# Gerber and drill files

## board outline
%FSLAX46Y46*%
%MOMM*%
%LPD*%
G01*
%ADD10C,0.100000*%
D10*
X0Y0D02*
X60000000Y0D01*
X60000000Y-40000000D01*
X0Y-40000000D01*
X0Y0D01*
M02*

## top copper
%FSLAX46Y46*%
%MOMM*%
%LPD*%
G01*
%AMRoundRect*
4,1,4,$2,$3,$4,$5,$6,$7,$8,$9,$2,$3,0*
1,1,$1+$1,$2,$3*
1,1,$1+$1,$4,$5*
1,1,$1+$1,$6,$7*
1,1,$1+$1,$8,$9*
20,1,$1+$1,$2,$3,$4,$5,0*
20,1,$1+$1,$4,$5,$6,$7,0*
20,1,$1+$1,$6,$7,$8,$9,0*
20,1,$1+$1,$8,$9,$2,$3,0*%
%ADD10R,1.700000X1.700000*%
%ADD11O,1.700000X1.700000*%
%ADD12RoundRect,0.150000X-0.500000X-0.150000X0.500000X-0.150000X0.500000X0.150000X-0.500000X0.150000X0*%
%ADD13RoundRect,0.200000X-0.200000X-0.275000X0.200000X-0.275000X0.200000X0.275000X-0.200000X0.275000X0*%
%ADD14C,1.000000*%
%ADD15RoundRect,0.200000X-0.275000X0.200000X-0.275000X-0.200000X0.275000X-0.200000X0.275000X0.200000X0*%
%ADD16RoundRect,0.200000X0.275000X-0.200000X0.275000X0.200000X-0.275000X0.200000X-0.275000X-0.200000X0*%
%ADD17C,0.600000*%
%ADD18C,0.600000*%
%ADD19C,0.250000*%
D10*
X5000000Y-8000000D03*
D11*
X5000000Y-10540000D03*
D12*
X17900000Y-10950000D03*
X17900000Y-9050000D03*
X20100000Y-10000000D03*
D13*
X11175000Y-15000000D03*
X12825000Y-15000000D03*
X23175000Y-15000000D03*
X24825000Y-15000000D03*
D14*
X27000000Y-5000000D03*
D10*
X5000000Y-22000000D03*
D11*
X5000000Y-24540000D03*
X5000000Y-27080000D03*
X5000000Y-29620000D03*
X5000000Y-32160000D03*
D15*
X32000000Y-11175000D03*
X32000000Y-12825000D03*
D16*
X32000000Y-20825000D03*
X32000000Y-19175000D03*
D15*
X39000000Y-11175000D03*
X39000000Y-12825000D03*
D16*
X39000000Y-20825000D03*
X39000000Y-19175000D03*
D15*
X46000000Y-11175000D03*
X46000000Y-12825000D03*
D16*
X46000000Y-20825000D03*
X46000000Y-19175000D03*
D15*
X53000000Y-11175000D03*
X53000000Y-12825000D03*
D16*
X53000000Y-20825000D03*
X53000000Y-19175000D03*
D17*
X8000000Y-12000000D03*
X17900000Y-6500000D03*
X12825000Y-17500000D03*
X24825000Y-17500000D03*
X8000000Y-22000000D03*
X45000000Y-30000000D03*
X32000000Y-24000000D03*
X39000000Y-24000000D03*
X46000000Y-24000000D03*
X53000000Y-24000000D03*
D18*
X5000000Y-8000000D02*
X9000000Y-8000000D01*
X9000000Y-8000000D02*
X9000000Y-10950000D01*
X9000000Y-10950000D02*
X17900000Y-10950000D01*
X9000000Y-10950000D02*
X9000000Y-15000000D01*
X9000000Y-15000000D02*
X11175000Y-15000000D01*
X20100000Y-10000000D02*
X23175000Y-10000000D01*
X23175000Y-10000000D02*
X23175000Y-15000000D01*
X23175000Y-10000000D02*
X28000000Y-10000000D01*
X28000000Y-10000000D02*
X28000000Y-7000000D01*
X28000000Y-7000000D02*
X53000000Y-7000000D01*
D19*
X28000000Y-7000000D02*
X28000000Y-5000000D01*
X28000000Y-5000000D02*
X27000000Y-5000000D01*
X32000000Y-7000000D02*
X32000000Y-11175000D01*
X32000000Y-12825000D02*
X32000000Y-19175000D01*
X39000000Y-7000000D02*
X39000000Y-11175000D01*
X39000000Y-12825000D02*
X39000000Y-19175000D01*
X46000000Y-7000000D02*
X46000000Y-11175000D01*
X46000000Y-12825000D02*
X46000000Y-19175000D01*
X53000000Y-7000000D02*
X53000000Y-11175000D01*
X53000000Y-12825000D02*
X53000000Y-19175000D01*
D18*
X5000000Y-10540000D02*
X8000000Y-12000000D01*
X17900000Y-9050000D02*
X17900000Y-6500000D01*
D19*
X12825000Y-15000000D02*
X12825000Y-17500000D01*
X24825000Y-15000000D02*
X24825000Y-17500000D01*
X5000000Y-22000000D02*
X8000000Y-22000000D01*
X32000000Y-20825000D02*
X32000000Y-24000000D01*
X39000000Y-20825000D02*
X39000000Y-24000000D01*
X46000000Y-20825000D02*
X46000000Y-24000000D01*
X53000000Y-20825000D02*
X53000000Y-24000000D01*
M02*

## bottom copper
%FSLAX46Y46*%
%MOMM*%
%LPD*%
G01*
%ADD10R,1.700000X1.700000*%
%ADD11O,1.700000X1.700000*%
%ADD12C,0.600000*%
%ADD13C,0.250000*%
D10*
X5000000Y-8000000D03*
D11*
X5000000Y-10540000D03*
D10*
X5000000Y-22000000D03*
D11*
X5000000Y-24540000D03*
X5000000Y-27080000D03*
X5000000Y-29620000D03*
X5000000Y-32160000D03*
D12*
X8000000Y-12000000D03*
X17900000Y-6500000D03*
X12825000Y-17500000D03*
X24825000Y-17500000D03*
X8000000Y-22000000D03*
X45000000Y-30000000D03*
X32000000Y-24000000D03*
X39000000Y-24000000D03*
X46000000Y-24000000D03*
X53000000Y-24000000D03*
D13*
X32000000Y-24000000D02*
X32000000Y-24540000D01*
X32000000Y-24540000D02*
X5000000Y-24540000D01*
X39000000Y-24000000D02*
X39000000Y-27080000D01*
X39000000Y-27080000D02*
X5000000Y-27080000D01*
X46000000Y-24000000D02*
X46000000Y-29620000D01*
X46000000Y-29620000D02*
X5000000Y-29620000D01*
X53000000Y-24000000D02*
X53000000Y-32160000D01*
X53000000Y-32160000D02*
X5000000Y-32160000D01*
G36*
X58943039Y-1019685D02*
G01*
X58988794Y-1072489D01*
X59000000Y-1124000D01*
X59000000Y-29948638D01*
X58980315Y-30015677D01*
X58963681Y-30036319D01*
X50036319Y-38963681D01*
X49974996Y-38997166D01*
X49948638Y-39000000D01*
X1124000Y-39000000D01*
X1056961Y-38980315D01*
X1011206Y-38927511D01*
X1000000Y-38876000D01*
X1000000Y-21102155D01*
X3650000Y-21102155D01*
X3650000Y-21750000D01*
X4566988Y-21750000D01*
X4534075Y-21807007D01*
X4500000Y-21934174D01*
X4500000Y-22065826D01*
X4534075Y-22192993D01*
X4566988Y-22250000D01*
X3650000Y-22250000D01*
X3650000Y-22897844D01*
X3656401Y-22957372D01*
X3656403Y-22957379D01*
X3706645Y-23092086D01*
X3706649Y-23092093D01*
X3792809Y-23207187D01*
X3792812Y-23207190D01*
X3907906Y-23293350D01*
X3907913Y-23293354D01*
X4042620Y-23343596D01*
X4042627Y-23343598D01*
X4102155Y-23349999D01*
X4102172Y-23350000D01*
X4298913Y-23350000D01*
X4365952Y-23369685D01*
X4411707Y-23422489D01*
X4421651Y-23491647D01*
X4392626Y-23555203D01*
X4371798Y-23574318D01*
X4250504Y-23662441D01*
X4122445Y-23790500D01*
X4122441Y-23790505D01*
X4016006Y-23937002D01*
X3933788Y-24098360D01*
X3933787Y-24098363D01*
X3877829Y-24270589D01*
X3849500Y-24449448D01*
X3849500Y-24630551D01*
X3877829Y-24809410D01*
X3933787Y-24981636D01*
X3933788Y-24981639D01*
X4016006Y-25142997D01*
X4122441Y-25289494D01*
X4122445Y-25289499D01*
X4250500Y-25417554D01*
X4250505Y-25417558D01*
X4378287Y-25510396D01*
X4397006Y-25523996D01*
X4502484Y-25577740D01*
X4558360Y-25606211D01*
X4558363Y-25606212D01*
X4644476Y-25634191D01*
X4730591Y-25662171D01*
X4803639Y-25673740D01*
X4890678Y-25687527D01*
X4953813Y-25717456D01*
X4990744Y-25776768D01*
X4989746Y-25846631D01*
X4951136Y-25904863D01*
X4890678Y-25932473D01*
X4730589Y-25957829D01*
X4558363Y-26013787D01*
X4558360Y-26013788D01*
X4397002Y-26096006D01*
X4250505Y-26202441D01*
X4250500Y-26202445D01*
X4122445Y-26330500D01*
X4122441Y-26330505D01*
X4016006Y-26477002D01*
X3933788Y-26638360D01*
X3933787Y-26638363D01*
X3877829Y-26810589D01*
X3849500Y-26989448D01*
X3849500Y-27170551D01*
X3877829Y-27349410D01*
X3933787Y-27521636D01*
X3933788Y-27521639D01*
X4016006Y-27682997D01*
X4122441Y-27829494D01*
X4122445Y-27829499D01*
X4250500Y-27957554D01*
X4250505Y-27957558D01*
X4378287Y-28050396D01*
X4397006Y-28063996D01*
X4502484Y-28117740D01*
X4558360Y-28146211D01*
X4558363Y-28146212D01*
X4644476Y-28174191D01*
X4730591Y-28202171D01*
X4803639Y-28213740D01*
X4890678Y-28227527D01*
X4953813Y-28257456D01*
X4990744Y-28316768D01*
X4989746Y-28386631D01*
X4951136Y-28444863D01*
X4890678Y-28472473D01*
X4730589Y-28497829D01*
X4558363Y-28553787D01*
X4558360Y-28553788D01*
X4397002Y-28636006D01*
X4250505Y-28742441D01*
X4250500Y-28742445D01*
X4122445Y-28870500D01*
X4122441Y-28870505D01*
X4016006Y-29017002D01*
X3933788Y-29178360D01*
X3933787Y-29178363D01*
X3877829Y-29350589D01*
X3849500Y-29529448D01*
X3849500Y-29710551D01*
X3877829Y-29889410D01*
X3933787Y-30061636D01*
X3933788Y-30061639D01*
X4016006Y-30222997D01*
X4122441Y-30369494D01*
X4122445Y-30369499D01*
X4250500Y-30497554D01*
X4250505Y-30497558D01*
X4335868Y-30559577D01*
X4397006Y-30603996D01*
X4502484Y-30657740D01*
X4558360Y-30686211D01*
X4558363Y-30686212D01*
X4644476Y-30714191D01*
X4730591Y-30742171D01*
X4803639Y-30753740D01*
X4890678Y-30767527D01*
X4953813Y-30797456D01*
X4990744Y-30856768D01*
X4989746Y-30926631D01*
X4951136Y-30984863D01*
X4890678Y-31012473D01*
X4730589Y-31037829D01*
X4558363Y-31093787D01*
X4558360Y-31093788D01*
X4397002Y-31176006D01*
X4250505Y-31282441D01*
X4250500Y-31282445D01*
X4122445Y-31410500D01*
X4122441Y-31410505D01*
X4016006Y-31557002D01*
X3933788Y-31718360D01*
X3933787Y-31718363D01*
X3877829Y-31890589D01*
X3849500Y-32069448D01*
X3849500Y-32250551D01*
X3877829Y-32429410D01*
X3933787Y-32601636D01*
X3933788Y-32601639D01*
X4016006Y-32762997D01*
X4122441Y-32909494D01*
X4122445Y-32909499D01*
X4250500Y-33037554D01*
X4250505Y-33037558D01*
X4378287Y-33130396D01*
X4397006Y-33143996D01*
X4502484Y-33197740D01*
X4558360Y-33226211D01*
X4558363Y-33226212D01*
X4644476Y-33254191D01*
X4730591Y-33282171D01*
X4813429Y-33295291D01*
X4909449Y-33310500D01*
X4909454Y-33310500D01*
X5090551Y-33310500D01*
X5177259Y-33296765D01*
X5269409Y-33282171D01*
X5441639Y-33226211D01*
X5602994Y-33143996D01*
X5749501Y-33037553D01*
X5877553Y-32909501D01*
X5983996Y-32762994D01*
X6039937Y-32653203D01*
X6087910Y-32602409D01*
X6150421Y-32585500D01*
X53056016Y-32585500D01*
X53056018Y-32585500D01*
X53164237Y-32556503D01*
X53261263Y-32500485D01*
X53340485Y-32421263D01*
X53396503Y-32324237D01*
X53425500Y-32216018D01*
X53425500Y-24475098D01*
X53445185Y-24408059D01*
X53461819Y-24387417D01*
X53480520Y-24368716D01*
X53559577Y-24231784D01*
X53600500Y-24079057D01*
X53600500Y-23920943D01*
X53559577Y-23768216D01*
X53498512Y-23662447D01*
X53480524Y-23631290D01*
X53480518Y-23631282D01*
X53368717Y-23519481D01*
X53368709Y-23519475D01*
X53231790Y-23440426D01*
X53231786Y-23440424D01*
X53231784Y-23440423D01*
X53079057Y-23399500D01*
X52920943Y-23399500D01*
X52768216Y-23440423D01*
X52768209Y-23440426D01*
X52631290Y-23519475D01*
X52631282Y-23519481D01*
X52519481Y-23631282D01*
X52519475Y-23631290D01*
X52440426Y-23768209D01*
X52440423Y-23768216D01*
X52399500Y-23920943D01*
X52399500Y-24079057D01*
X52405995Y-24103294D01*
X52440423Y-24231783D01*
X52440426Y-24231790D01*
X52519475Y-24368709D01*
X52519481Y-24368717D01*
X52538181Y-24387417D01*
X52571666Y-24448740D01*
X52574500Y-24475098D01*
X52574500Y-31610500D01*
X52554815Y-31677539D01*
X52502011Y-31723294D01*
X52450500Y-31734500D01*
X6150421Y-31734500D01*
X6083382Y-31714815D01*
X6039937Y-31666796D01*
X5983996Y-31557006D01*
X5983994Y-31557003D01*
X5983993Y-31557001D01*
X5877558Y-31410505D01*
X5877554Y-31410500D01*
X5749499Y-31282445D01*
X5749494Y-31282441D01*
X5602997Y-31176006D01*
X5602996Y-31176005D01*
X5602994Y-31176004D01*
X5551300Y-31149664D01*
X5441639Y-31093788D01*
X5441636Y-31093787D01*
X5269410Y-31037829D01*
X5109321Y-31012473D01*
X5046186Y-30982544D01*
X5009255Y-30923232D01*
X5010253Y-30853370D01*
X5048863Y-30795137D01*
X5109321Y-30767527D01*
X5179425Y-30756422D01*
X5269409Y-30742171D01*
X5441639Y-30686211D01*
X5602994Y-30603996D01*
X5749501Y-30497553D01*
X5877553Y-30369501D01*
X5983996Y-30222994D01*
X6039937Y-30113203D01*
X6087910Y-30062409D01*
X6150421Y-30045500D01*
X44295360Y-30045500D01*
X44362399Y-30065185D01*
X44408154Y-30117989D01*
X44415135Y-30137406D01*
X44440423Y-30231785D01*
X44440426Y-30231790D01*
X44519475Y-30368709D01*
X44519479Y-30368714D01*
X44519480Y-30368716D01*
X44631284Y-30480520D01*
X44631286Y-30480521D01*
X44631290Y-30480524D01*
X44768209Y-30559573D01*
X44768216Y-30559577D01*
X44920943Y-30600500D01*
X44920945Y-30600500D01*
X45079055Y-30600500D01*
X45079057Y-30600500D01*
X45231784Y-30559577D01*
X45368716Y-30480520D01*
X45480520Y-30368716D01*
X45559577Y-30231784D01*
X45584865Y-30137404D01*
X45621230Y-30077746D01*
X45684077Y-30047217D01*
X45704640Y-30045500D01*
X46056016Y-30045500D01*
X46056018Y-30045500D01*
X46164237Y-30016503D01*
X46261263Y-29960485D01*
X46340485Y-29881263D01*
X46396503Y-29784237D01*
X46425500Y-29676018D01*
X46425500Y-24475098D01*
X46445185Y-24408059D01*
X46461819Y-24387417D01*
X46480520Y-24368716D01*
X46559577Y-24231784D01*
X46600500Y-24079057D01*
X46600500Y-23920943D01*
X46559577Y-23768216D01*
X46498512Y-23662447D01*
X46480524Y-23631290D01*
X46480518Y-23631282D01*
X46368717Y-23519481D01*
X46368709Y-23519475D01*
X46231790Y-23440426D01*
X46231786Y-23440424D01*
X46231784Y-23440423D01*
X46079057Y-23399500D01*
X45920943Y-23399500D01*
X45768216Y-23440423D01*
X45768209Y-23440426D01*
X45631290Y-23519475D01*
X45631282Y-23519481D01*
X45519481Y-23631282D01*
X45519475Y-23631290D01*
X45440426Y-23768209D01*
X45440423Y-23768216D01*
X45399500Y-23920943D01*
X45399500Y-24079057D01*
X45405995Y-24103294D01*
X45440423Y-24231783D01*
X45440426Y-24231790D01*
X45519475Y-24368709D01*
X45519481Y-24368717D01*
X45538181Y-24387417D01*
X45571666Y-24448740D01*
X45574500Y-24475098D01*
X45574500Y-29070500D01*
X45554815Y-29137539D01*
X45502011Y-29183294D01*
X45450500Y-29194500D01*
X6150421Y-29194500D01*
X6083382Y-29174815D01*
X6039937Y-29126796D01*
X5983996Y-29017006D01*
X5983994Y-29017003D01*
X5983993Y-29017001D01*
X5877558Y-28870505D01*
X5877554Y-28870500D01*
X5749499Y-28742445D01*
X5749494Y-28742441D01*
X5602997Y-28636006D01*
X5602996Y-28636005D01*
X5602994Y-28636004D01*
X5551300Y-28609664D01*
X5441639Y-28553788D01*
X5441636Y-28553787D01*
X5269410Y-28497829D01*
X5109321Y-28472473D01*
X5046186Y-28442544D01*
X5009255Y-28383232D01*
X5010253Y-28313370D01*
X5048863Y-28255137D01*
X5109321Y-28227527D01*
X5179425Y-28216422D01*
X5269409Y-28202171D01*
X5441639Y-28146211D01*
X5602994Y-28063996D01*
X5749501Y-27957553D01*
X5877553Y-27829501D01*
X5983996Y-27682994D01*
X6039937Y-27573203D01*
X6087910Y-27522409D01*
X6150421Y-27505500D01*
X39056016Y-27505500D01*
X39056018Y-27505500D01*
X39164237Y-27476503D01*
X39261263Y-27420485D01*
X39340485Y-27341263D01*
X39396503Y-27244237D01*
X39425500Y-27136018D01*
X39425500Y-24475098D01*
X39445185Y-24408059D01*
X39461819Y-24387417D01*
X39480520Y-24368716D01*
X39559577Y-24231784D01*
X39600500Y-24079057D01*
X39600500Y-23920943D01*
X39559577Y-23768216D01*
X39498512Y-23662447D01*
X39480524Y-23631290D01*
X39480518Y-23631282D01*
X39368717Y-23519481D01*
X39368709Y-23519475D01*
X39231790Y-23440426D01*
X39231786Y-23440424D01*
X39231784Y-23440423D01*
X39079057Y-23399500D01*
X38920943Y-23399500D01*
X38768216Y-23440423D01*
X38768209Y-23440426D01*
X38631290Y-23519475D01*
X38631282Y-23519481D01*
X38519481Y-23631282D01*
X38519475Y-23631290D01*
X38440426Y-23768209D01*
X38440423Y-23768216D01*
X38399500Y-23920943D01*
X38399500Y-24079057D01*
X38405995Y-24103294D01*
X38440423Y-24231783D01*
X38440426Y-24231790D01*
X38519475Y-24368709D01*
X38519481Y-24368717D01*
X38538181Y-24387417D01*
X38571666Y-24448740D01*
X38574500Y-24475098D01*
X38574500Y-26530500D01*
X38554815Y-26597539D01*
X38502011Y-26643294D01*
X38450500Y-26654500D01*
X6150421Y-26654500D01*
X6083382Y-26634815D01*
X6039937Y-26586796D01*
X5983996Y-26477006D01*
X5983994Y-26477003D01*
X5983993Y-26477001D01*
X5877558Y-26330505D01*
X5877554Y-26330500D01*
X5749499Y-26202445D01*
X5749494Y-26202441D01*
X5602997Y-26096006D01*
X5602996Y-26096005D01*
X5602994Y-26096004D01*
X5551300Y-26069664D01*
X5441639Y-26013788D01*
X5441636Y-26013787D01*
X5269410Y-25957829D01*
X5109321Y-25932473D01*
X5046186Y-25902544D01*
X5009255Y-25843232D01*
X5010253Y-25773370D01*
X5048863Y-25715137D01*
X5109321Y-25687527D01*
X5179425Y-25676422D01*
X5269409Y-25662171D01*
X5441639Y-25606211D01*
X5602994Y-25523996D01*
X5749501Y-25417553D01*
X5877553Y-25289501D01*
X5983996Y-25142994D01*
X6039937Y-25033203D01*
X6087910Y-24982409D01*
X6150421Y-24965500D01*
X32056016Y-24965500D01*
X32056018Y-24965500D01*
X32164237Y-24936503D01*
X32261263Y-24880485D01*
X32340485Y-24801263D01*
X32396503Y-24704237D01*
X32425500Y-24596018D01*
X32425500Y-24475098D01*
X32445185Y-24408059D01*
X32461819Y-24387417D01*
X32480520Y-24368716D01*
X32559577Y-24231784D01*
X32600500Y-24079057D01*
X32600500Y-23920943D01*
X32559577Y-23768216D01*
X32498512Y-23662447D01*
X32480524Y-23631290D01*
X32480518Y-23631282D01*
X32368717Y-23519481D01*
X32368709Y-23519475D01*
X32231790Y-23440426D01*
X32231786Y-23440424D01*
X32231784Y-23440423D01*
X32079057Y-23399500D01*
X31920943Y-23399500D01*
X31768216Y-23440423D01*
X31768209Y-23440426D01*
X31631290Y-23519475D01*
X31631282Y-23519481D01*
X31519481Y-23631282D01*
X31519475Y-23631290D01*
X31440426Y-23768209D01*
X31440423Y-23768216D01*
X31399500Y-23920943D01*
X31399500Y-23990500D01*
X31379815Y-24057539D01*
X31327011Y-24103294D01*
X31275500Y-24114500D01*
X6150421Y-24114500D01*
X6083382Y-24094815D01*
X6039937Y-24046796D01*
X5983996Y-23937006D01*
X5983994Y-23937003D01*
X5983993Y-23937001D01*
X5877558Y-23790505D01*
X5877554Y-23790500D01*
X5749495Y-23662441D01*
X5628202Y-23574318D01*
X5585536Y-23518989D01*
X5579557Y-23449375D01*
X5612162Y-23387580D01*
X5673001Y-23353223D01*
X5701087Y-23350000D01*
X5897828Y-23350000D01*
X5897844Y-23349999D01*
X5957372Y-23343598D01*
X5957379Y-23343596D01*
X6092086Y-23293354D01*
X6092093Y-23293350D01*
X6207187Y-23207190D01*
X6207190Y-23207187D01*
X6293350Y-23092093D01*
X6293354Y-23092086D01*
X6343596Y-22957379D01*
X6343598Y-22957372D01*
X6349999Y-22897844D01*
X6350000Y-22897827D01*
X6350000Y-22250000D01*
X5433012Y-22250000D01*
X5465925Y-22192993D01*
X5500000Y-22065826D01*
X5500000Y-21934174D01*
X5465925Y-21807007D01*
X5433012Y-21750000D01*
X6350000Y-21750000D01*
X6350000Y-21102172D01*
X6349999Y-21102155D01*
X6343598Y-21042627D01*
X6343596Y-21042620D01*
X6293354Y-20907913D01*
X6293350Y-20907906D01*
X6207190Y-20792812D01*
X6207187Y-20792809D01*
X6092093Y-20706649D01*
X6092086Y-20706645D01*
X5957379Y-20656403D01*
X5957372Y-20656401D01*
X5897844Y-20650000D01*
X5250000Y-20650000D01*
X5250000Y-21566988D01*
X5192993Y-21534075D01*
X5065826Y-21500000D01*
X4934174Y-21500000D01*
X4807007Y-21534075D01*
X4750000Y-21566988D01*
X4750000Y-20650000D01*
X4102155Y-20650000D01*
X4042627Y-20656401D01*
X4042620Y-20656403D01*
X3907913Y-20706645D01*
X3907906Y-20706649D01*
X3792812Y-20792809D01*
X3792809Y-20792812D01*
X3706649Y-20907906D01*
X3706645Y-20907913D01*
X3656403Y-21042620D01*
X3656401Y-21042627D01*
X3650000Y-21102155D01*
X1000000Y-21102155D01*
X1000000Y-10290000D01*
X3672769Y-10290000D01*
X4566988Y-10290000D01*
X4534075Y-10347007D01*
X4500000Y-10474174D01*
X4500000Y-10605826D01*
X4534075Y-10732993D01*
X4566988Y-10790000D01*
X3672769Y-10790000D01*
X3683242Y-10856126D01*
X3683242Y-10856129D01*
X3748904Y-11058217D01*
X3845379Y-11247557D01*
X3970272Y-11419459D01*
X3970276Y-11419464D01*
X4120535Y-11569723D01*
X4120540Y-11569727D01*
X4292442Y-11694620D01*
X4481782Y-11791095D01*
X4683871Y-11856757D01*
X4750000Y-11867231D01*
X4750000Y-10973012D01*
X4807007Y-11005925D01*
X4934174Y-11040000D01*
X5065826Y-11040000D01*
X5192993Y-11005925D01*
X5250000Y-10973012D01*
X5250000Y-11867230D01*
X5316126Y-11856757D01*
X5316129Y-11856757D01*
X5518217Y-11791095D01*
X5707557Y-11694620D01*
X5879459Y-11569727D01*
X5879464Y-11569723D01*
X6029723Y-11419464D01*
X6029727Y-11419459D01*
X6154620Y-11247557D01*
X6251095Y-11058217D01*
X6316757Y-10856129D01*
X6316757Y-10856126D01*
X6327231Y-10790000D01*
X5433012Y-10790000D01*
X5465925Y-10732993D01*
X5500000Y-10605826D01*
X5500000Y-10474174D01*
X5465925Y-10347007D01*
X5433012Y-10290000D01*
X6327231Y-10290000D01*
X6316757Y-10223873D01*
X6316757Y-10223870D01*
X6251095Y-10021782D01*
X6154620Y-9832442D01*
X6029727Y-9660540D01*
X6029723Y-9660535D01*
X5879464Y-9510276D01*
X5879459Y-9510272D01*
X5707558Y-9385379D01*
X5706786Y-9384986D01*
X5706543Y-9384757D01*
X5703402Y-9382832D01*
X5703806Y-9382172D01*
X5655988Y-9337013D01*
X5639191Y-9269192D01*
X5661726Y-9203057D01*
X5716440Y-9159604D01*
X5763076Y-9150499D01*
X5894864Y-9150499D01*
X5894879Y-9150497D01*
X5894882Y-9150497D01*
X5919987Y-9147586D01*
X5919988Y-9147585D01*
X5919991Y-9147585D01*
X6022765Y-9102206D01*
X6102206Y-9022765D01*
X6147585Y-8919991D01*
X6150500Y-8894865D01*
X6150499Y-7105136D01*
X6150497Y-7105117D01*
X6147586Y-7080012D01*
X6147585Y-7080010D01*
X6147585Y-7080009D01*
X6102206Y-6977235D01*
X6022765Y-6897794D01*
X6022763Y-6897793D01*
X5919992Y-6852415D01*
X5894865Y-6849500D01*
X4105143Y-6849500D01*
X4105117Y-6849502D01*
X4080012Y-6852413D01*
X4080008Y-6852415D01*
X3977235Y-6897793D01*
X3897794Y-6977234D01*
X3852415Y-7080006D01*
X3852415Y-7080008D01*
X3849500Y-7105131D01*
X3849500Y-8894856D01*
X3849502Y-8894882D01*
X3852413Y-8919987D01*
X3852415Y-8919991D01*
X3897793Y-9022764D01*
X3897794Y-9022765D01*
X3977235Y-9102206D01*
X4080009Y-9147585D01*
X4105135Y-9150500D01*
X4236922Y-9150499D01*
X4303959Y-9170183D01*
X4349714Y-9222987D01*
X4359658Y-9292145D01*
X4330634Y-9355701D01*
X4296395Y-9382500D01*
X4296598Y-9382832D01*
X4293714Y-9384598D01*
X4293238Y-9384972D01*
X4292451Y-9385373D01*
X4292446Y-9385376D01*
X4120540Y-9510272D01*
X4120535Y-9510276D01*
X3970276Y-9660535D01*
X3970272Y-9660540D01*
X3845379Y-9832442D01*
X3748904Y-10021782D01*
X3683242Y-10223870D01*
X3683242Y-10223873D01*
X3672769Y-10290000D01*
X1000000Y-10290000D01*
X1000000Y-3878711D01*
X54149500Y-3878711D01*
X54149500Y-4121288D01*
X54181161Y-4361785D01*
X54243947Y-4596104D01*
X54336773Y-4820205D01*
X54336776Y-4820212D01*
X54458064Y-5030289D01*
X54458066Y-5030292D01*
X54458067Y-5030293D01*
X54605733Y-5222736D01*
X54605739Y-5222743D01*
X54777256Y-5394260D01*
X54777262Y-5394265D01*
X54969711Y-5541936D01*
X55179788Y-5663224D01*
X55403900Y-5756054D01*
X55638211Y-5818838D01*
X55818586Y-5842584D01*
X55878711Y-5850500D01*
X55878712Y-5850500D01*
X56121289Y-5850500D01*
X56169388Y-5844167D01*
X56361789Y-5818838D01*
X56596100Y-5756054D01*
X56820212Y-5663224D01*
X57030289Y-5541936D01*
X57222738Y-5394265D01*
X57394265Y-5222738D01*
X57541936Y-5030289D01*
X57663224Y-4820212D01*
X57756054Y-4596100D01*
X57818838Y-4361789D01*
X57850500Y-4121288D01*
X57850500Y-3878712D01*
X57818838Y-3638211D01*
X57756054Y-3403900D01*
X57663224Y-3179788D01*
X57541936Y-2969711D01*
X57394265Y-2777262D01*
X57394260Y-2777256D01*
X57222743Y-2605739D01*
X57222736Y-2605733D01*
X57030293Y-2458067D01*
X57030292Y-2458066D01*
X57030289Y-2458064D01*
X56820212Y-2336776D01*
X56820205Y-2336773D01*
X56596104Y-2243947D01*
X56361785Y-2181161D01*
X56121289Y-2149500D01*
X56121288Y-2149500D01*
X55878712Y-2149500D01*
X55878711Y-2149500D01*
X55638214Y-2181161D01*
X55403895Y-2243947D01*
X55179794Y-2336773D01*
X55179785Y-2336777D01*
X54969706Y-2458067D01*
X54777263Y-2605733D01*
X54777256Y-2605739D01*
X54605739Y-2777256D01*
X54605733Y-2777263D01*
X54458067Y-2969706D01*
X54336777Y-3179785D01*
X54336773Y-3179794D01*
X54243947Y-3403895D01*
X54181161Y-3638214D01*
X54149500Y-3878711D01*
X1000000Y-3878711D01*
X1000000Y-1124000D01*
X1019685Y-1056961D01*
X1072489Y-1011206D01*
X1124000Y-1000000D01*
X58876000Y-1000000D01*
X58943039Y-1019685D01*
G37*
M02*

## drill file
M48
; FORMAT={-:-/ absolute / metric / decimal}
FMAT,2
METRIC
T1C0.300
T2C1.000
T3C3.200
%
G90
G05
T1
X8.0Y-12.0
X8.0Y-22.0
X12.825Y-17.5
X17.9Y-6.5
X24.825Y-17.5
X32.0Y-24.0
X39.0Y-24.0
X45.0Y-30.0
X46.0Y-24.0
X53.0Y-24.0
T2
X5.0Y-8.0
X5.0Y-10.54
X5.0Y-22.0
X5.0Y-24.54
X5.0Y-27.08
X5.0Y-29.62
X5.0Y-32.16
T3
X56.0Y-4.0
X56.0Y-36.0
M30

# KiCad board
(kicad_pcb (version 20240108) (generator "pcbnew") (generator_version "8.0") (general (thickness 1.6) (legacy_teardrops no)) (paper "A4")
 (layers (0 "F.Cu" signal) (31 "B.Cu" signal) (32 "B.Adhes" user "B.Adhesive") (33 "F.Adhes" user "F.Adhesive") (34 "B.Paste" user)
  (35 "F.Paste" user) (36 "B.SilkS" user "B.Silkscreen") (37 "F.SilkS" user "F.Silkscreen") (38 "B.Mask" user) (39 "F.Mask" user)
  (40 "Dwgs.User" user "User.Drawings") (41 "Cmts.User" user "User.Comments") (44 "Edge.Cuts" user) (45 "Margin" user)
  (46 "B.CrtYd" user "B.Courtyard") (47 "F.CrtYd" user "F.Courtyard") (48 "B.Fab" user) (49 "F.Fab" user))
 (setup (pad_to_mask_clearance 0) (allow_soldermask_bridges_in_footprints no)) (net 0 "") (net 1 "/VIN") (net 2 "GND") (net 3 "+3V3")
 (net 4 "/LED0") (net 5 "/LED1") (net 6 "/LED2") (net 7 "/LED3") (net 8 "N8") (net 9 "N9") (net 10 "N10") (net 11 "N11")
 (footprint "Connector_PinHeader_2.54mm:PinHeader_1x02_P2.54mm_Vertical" (layer "F.Cu") (at 5 8)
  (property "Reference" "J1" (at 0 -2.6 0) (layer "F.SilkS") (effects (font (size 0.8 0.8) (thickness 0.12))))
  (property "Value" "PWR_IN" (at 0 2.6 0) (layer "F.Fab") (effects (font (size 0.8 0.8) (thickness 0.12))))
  (pad "1" thru_hole rect (at 0 0) (size 1.7 1.7) (drill 1) (layers "*.Cu" "*.Mask") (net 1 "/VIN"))
  (pad "2" thru_hole oval (at 0 2.54) (size 1.7 1.7) (drill 1) (layers "*.Cu" "*.Mask") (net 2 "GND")))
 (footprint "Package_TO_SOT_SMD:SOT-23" (layer "F.Cu") (at 19 10)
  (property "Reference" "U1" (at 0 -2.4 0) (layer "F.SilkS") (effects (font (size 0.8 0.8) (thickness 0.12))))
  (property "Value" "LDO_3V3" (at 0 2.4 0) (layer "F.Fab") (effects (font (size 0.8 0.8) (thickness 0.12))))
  (pad "1" smd roundrect (at -1.1 0.95) (size 1.3 0.6) (layers "F.Cu" "F.Paste" "F.Mask") (roundrect_rratio 0.25) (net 1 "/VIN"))
  (pad "2" smd roundrect (at -1.1 -0.95) (size 1.3 0.6) (layers "F.Cu" "F.Paste" "F.Mask") (roundrect_rratio 0.25) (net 2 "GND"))
  (pad "3" smd roundrect (at 1.1 0) (size 1.3 0.6) (layers "F.Cu" "F.Paste" "F.Mask") (roundrect_rratio 0.25) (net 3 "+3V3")))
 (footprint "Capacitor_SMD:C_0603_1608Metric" (layer "F.Cu") (at 12 15)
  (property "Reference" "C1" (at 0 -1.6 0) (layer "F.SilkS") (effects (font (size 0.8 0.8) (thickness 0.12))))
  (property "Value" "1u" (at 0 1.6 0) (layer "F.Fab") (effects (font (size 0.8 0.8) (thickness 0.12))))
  (pad "1" smd roundrect (at -0.825 0) (size 0.8 0.95) (layers "F.Cu" "F.Paste" "F.Mask") (roundrect_rratio 0.25) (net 1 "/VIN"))
  (pad "2" smd roundrect (at 0.825 0) (size 0.8 0.95) (layers "F.Cu" "F.Paste" "F.Mask") (roundrect_rratio 0.25) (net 2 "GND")))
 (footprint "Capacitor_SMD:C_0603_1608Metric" (layer "F.Cu") (at 24 15)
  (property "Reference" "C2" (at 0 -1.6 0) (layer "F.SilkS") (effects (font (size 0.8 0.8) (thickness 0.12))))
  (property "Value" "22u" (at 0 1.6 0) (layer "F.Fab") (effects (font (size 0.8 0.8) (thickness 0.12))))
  (pad "1" smd roundrect (at -0.825 0) (size 0.8 0.95) (layers "F.Cu" "F.Paste" "F.Mask") (roundrect_rratio 0.25) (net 3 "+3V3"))
  (pad "2" smd roundrect (at 0.825 0) (size 0.8 0.95) (layers "F.Cu" "F.Paste" "F.Mask") (roundrect_rratio 0.25) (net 2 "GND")))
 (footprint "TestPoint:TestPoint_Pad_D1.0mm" (layer "F.Cu") (at 27 5)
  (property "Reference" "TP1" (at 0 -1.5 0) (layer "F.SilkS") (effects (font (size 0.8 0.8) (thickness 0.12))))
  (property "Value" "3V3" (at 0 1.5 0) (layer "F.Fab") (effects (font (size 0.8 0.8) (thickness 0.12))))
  (pad "1" smd circle (at 0 0) (size 1 1) (layers "F.Cu" "F.Mask") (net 3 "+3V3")))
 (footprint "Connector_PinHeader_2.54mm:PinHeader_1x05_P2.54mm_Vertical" (layer "F.Cu") (at 5 22)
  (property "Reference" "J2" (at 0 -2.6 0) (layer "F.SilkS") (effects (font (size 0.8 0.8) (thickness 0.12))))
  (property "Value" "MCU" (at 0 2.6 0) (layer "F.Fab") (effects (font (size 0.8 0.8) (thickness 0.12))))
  (pad "1" thru_hole rect (at 0 0) (size 1.7 1.7) (drill 1) (layers "*.Cu" "*.Mask") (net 2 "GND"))
  (pad "2" thru_hole oval (at 0 2.54) (size 1.7 1.7) (drill 1) (layers "*.Cu" "*.Mask") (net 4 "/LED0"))
  (pad "3" thru_hole oval (at 0 5.08) (size 1.7 1.7) (drill 1) (layers "*.Cu" "*.Mask") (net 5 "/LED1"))
  (pad "4" thru_hole oval (at 0 7.62) (size 1.7 1.7) (drill 1) (layers "*.Cu" "*.Mask") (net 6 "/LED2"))
  (pad "5" thru_hole oval (at 0 10.16) (size 1.7 1.7) (drill 1) (layers "*.Cu" "*.Mask") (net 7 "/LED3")))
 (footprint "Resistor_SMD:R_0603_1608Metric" (layer "F.Cu") (at 32 12 270)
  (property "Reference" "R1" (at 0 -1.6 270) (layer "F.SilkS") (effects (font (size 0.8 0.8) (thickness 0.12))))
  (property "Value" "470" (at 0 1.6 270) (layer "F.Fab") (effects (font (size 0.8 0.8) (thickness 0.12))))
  (pad "1" smd roundrect (at -0.825 0 270) (size 0.8 0.95) (layers "F.Cu" "F.Paste" "F.Mask") (roundrect_rratio 0.25) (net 3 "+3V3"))
  (pad "2" smd roundrect (at 0.825 0 270) (size 0.8 0.95) (layers "F.Cu" "F.Paste" "F.Mask") (roundrect_rratio 0.25) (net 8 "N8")))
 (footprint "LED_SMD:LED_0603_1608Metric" (layer "F.Cu") (at 32 20 90)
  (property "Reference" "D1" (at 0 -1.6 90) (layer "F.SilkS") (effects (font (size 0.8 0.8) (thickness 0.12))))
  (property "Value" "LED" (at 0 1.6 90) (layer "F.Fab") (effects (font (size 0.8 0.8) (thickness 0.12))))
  (pad "1" smd roundrect (at -0.825 0 90) (size 0.8 0.95) (layers "F.Cu" "F.Paste" "F.Mask") (roundrect_rratio 0.25) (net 4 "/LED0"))
  (pad "2" smd roundrect (at 0.825 0 90) (size 0.8 0.95) (layers "F.Cu" "F.Paste" "F.Mask") (roundrect_rratio 0.25) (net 8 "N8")))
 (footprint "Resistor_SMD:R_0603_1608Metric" (layer "F.Cu") (at 39 12 270)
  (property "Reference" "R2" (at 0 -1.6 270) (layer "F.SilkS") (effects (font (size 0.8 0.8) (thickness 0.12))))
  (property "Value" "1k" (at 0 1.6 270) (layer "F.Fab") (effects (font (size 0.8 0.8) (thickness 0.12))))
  (pad "1" smd roundrect (at -0.825 0 270) (size 0.8 0.95) (layers "F.Cu" "F.Paste" "F.Mask") (roundrect_rratio 0.25) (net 3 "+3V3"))
  (pad "2" smd roundrect (at 0.825 0 270) (size 0.8 0.95) (layers "F.Cu" "F.Paste" "F.Mask") (roundrect_rratio 0.25) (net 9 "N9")))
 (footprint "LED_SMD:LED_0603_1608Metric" (layer "F.Cu") (at 39 20 90)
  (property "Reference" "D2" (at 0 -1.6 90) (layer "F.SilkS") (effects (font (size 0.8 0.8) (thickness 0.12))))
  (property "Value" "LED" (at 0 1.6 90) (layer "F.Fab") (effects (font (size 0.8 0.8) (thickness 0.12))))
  (pad "1" smd roundrect (at -0.825 0 90) (size 0.8 0.95) (layers "F.Cu" "F.Paste" "F.Mask") (roundrect_rratio 0.25) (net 5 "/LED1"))
  (pad "2" smd roundrect (at 0.825 0 90) (size 0.8 0.95) (layers "F.Cu" "F.Paste" "F.Mask") (roundrect_rratio 0.25) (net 9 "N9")))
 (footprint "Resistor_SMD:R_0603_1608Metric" (layer "F.Cu") (at 46 12 270)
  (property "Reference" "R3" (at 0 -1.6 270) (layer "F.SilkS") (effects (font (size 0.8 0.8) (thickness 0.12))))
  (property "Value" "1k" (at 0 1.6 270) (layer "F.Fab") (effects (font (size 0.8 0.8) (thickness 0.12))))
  (pad "1" smd roundrect (at -0.825 0 270) (size 0.8 0.95) (layers "F.Cu" "F.Paste" "F.Mask") (roundrect_rratio 0.25) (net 3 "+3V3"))
  (pad "2" smd roundrect (at 0.825 0 270) (size 0.8 0.95) (layers "F.Cu" "F.Paste" "F.Mask") (roundrect_rratio 0.25) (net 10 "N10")))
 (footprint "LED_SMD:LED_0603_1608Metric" (layer "F.Cu") (at 46 20 90)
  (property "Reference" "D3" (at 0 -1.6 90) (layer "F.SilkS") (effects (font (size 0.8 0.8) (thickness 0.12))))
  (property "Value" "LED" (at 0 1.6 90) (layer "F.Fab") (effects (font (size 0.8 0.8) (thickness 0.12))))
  (pad "1" smd roundrect (at -0.825 0 90) (size 0.8 0.95) (layers "F.Cu" "F.Paste" "F.Mask") (roundrect_rratio 0.25) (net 6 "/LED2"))
  (pad "2" smd roundrect (at 0.825 0 90) (size 0.8 0.95) (layers "F.Cu" "F.Paste" "F.Mask") (roundrect_rratio 0.25) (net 10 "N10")))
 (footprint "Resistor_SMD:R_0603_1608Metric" (layer "F.Cu") (at 53 12 270)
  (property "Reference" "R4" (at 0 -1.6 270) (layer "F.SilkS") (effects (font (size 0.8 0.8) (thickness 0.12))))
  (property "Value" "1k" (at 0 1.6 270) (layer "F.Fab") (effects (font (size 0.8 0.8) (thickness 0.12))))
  (pad "1" smd roundrect (at -0.825 0 270) (size 0.8 0.95) (layers "F.Cu" "F.Paste" "F.Mask") (roundrect_rratio 0.25) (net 3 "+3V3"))
  (pad "2" smd roundrect (at 0.825 0 270) (size 0.8 0.95) (layers "F.Cu" "F.Paste" "F.Mask") (roundrect_rratio 0.25) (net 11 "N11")))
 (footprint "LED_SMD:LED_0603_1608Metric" (layer "F.Cu") (at 53 20 90)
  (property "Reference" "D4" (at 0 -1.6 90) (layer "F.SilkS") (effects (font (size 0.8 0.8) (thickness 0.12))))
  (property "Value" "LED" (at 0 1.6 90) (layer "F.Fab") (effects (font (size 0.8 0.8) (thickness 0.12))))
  (pad "1" smd roundrect (at -0.825 0 90) (size 0.8 0.95) (layers "F.Cu" "F.Paste" "F.Mask") (roundrect_rratio 0.25) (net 7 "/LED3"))
  (pad "2" smd roundrect (at 0.825 0 90) (size 0.8 0.95) (layers "F.Cu" "F.Paste" "F.Mask") (roundrect_rratio 0.25) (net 11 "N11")))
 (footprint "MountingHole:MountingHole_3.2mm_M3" (layer "F.Cu") (at 56 4)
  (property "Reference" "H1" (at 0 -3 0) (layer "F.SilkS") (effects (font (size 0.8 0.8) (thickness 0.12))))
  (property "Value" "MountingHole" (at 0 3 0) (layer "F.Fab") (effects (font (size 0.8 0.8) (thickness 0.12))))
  (pad "" np_thru_hole circle (at 0 0) (size 3.2 3.2) (drill 3.2) (layers "*.Cu" "*.Mask")))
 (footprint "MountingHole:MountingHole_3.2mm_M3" (layer "F.Cu") (at 56 36)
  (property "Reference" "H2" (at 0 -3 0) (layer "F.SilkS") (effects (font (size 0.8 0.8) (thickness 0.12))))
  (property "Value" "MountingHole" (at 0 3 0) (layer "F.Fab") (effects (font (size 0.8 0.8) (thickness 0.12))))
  (pad "" np_thru_hole circle (at 0 0) (size 3.2 3.2) (drill 3.2) (layers "*.Cu" "*.Mask")))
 (segment (start 5 8) (end 9 8) (width 0.6) (layer "F.Cu") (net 1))
 (segment (start 9 8) (end 9 10.95) (width 0.6) (layer "F.Cu") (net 1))
 (segment (start 9 10.95) (end 17.9 10.95) (width 0.6) (layer "F.Cu") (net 1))
 (segment (start 9 10.95) (end 9 15) (width 0.6) (layer "F.Cu") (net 1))
 (segment (start 9 15) (end 11.175 15) (width 0.6) (layer "F.Cu") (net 1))
 (segment (start 20.1 10) (end 23.175 10) (width 0.6) (layer "F.Cu") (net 3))
 (segment (start 23.175 10) (end 23.175 15) (width 0.6) (layer "F.Cu") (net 3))
 (segment (start 23.175 10) (end 28 10) (width 0.6) (layer "F.Cu") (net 3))
 (segment (start 28 10) (end 28 7) (width 0.6) (layer "F.Cu") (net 3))
 (segment (start 28 7) (end 53 7) (width 0.6) (layer "F.Cu") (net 3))
 (segment (start 28 7) (end 28 5) (width 0.25) (layer "F.Cu") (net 3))
 (segment (start 28 5) (end 27 5) (width 0.25) (layer "F.Cu") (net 3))
 (segment (start 32 7) (end 32 11.175) (width 0.25) (layer "F.Cu") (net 3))
 (segment (start 32 12.825) (end 32 19.175) (width 0.25) (layer "F.Cu") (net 8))
 (segment (start 39 7) (end 39 11.175) (width 0.25) (layer "F.Cu") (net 3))
 (segment (start 39 12.825) (end 39 19.175) (width 0.25) (layer "F.Cu") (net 9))
 (segment (start 46 7) (end 46 11.175) (width 0.25) (layer "F.Cu") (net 3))
 (segment (start 46 12.825) (end 46 19.175) (width 0.25) (layer "F.Cu") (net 10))
 (segment (start 53 7) (end 53 11.175) (width 0.25) (layer "F.Cu") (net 3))
 (segment (start 53 12.825) (end 53 19.175) (width 0.25) (layer "F.Cu") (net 11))
 (segment (start 5 10.54) (end 8 12) (width 0.6) (layer "F.Cu") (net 2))
 (via (at 8 12) (size 0.6) (drill 0.3) (layers "F.Cu" "B.Cu") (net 2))
 (segment (start 17.9 9.05) (end 17.9 6.5) (width 0.6) (layer "F.Cu") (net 2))
 (via (at 17.9 6.5) (size 0.6) (drill 0.3) (layers "F.Cu" "B.Cu") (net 2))
 (segment (start 12.825 15) (end 12.825 17.5) (width 0.25) (layer "F.Cu") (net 2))
 (via (at 12.825 17.5) (size 0.6) (drill 0.3) (layers "F.Cu" "B.Cu") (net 2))
 (segment (start 24.825 15) (end 24.825 17.5) (width 0.25) (layer "F.Cu") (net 2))
 (via (at 24.825 17.5) (size 0.6) (drill 0.3) (layers "F.Cu" "B.Cu") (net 2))
 (segment (start 5 22) (end 8 22) (width 0.25) (layer "F.Cu") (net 2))
 (via (at 8 22) (size 0.6) (drill 0.3) (layers "F.Cu" "B.Cu") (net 2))
 (via (at 45 30) (size 0.6) (drill 0.3) (layers "F.Cu" "B.Cu") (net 2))
 (segment (start 32 20.825) (end 32 24) (width 0.25) (layer "F.Cu") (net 4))
 (via (at 32 24) (size 0.6) (drill 0.3) (layers "F.Cu" "B.Cu") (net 4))
 (segment (start 32 24) (end 32 24.54) (width 0.25) (layer "B.Cu") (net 4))
 (segment (start 32 24.54) (end 5 24.54) (width 0.25) (layer "B.Cu") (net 4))
 (segment (start 39 20.825) (end 39 24) (width 0.25) (layer "F.Cu") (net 5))
 (via (at 39 24) (size 0.6) (drill 0.3) (layers "F.Cu" "B.Cu") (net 5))
 (segment (start 39 24) (end 39 27.08) (width 0.25) (layer "B.Cu") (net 5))
 (segment (start 39 27.08) (end 5 27.08) (width 0.25) (layer "B.Cu") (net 5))
 (segment (start 46 20.825) (end 46 24) (width 0.25) (layer "F.Cu") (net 6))
 (via (at 46 24) (size 0.6) (drill 0.3) (layers "F.Cu" "B.Cu") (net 6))
 (segment (start 46 24) (end 46 29.62) (width 0.25) (layer "B.Cu") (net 6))
 (segment (start 46 29.62) (end 5 29.62) (width 0.25) (layer "B.Cu") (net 6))
 (segment (start 53 20.825) (end 53 24) (width 0.25) (layer "F.Cu") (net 7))
 (via (at 53 24) (size 0.6) (drill 0.3) (layers "F.Cu" "B.Cu") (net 7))
 (segment (start 53 24) (end 53 32.16) (width 0.25) (layer "B.Cu") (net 7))
 (segment (start 53 32.16) (end 5 32.16) (width 0.25) (layer "B.Cu") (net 7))
 (gr_rect (start 0 0) (end 60 40) (stroke (width 0.1) (type default)) (fill none) (layer "Edge.Cuts"))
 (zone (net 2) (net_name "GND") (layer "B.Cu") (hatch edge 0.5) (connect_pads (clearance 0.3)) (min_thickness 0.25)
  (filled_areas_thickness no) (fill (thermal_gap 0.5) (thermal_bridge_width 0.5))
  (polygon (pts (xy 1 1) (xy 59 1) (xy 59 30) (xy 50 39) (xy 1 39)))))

